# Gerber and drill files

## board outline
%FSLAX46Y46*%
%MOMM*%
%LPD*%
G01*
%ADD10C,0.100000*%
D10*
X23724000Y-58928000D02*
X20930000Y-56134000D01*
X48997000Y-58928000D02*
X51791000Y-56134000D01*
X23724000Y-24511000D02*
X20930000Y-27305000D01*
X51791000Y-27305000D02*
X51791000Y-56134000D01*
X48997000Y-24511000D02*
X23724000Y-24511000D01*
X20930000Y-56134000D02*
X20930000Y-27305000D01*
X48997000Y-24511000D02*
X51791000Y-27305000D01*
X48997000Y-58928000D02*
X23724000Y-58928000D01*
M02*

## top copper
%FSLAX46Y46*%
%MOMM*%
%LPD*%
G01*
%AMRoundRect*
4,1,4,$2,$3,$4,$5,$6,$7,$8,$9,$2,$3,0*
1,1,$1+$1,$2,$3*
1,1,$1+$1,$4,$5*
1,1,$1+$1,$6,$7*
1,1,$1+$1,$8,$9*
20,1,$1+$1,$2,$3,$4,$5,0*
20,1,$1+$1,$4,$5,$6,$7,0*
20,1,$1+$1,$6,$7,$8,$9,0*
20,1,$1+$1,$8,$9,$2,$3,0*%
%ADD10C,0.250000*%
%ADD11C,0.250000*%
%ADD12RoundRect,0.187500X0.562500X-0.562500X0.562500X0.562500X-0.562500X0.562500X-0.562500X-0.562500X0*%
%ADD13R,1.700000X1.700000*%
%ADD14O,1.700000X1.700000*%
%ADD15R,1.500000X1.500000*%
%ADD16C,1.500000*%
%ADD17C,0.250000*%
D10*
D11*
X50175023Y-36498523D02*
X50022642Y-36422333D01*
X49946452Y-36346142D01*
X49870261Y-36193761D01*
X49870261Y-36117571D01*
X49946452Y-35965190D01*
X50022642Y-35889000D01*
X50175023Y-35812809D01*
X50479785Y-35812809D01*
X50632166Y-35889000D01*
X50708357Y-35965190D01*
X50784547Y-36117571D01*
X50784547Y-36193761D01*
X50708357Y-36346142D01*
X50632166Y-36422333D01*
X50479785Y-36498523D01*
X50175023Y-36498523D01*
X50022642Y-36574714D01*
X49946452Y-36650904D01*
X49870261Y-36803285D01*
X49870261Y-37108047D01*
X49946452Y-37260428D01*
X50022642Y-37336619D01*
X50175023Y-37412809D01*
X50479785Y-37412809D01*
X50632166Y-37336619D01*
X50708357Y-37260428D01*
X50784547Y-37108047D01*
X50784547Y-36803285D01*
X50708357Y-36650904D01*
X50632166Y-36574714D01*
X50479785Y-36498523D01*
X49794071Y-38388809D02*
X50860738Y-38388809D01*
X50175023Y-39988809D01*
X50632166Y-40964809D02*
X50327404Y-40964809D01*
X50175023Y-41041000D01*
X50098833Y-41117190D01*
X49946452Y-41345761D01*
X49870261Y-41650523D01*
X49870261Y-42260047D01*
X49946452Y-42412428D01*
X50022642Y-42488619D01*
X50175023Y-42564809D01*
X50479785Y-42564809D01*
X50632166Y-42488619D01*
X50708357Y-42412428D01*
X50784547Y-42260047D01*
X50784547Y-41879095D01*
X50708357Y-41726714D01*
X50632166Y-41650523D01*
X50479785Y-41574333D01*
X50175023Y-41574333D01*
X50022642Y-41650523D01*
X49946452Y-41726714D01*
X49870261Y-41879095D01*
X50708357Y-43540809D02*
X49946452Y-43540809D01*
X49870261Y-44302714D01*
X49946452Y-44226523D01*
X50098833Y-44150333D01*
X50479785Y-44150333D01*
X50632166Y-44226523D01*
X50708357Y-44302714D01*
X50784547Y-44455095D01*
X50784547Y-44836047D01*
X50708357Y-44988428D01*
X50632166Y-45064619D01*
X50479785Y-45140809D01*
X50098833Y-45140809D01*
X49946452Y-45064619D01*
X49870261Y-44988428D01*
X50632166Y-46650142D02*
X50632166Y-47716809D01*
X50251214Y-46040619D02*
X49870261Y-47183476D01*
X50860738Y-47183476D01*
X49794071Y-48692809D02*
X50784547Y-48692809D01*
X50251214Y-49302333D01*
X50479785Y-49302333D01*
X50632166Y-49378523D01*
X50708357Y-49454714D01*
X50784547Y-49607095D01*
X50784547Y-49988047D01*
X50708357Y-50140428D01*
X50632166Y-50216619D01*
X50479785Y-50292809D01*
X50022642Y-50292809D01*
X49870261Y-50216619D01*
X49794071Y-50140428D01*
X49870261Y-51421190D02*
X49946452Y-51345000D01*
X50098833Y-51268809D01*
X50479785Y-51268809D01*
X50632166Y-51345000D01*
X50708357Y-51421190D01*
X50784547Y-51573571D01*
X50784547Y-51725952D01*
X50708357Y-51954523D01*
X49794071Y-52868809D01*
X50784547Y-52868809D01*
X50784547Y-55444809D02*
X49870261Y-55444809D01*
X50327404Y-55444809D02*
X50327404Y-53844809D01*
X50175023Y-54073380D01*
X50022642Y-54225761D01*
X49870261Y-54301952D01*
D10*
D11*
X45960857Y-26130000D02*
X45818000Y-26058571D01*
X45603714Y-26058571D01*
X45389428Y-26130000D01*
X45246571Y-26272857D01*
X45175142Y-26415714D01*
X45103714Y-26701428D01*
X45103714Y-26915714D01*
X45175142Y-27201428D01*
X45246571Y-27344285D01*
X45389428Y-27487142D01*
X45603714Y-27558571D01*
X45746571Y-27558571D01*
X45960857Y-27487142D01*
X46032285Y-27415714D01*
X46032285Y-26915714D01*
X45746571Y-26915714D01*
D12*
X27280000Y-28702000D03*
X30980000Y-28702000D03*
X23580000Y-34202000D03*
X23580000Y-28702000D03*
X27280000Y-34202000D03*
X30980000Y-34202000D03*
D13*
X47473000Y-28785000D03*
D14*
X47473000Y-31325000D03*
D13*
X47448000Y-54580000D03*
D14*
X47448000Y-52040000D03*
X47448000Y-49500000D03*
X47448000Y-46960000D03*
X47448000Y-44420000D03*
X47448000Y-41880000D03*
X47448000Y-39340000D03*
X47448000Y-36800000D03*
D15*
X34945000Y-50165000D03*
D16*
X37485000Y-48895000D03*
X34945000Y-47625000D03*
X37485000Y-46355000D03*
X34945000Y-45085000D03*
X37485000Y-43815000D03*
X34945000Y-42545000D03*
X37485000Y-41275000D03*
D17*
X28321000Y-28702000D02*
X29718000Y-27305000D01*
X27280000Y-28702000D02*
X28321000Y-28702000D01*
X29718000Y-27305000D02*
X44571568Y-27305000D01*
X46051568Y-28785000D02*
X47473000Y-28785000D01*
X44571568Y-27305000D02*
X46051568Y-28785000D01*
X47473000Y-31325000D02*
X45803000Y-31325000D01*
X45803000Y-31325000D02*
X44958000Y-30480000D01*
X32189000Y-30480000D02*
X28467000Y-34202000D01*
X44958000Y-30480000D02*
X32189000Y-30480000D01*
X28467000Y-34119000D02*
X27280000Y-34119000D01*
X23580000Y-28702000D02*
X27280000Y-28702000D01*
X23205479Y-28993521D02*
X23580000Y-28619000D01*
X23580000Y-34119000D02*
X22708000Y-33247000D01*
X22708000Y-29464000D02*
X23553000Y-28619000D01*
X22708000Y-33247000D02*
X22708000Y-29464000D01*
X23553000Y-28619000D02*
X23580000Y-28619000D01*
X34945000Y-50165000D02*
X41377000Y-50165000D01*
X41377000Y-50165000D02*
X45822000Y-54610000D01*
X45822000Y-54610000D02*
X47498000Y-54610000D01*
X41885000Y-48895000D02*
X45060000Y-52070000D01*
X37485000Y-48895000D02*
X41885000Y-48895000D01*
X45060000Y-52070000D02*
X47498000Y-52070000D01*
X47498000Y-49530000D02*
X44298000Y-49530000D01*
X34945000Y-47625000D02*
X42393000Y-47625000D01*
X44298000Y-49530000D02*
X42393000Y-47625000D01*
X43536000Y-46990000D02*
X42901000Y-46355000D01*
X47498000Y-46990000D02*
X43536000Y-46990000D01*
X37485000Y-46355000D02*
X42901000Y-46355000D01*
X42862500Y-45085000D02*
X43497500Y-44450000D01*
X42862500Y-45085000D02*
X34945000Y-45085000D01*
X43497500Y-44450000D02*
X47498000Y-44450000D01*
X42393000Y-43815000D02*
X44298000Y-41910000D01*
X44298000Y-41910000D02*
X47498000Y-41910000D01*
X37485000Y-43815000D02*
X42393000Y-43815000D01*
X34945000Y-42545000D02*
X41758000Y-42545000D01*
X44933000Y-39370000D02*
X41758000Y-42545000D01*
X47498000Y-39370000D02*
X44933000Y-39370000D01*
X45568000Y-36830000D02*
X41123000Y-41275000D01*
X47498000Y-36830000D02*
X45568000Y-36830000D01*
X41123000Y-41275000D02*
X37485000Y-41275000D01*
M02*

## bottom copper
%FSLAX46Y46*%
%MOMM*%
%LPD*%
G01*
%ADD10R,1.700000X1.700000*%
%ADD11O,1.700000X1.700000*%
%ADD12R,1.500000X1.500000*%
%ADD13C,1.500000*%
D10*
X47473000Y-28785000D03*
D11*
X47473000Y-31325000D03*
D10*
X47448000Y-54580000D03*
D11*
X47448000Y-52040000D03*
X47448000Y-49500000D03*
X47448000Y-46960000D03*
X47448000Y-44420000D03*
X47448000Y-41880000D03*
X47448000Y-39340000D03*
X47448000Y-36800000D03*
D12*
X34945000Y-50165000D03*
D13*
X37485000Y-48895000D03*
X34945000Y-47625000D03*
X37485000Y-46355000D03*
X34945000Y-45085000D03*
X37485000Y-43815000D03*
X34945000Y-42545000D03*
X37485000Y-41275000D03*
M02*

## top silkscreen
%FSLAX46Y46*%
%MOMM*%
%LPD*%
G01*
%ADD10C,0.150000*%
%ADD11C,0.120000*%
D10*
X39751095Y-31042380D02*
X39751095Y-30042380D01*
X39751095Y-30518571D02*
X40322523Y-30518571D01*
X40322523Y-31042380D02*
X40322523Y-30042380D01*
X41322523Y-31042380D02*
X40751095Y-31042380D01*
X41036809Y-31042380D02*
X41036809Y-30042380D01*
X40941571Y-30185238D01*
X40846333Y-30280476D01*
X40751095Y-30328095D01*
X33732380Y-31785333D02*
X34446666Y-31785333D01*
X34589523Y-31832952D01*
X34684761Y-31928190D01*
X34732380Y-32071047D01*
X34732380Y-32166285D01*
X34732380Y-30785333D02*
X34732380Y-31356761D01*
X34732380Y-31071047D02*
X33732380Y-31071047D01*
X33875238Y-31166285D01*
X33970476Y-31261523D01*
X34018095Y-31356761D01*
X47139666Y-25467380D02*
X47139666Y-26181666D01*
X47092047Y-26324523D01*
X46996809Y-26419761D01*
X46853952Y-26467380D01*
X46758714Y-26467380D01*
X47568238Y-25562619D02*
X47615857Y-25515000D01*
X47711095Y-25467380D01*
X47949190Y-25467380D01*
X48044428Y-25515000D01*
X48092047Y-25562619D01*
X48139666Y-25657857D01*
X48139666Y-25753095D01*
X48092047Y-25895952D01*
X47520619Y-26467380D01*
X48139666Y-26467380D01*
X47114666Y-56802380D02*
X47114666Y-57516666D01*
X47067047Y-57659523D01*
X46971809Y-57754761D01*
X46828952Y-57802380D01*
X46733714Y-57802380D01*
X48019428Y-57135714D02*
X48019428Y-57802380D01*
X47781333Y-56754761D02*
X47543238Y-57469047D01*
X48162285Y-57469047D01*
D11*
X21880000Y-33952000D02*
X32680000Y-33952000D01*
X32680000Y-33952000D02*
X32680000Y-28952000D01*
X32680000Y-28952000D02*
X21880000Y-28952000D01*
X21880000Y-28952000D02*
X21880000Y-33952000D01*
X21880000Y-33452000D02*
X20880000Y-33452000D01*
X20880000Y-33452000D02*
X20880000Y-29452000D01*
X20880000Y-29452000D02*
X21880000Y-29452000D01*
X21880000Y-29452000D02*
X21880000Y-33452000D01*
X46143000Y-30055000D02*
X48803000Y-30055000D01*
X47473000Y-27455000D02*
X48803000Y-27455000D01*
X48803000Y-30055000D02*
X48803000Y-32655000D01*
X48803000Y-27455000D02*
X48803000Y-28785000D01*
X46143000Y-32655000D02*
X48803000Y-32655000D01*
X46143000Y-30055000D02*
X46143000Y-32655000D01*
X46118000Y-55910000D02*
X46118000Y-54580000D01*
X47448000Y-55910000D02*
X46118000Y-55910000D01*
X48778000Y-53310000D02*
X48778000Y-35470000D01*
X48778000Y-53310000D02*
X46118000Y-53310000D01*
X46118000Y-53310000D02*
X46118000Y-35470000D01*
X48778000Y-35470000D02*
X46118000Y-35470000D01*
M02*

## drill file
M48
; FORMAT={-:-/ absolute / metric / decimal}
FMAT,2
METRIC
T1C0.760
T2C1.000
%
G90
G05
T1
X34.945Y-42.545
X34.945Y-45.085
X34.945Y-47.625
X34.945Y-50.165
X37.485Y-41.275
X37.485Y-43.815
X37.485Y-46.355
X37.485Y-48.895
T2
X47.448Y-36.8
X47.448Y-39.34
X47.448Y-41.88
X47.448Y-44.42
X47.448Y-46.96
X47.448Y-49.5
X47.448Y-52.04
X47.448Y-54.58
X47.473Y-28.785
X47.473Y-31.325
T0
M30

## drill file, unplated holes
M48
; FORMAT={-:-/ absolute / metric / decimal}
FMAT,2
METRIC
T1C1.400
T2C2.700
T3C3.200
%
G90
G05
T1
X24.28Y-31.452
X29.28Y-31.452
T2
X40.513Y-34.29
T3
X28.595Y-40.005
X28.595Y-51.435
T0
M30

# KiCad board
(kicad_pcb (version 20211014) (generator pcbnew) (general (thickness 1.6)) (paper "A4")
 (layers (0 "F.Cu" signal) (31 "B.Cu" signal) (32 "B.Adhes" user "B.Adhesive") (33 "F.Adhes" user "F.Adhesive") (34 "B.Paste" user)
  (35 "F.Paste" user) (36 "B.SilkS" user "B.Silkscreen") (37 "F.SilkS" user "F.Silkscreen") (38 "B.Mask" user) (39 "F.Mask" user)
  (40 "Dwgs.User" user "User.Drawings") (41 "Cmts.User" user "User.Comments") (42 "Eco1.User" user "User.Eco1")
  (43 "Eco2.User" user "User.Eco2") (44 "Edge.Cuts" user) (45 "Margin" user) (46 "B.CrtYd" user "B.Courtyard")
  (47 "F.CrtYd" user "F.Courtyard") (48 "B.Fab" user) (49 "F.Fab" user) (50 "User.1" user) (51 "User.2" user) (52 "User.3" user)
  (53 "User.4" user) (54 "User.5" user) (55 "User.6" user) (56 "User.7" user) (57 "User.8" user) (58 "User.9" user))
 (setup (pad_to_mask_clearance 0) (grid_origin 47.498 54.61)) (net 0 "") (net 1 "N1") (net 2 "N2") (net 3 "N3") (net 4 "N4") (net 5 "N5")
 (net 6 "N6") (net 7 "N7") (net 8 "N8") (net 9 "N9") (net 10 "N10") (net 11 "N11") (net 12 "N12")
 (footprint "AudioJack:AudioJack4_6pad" (layer "F.Cu") (at 27.28 31.452 90)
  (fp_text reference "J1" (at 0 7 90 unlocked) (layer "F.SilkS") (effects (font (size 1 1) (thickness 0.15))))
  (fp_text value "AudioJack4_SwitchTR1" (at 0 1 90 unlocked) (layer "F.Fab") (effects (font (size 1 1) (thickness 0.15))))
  (fp_rect (start -2.5 -5.4) (end 2.5 5.4) (layer "F.SilkS") (width 0.12) (fill none))
  (fp_rect (start -2 -5.4) (end 2 -6.4) (layer "F.SilkS") (width 0.12) (fill none))
  (pad "" np_thru_hole circle (at 0 -3 90) (size 1.4 1.4) (drill 1.4) (layers F&B.Cu *.Mask))
  (pad "" np_thru_hole circle (at 0 2 90) (size 1.4 1.4) (drill 1.4) (layers F&B.Cu *.Mask))
  (pad "R1" smd roundrect (at 2.75 0 90) (size 1.5 1.5) (layers "F.Cu" "F.Paste" "F.Mask") (roundrect_rratio 0.125) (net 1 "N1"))
  (pad "R1N" smd roundrect (at 2.75 3.7 90) (size 1.5 1.5) (layers "F.Cu" "F.Paste" "F.Mask") (roundrect_rratio 0.125) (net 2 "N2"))
  (pad "R2" smd roundrect (at -2.75 -3.7 90) (size 1.5 1.5) (layers "F.Cu" "F.Paste" "F.Mask") (roundrect_rratio 0.125) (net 1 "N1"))
  (pad "S" smd roundrect (at 2.75 -3.7 90) (size 1.5 1.5) (layers "F.Cu" "F.Paste" "F.Mask") (roundrect_rratio 0.125) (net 1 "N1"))
  (pad "T" smd roundrect (at -2.75 0 90) (size 1.5 1.5) (layers "F.Cu" "F.Paste" "F.Mask") (roundrect_rratio 0.125) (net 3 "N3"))
  (pad "TN" smd roundrect (at -2.75 3.7 90) (size 1.5 1.5) (layers "F.Cu" "F.Paste" "F.Mask") (roundrect_rratio 0.125) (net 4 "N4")))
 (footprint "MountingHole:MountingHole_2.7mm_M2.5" (layer "F.Cu") (at 40.513 34.29)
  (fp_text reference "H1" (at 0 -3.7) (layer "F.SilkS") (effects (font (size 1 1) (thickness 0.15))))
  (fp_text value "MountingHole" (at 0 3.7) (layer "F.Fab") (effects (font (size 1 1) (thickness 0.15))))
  (pad "" np_thru_hole circle locked (at 0 0) (size 2.7 2.7) (drill 2.7) (layers *.Cu *.Mask)))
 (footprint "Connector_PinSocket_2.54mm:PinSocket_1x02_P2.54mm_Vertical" (layer "F.Cu") (at 47.473 28.785)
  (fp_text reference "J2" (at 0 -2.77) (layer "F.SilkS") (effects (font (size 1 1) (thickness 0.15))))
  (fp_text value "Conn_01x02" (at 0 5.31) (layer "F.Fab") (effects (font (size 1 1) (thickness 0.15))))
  (fp_line (start -1.33 1.27) (end 1.33 1.27) (layer "F.SilkS") (width 0.12))
  (fp_line (start 0 -1.33) (end 1.33 -1.33) (layer "F.SilkS") (width 0.12))
  (fp_line (start 1.33 1.27) (end 1.33 3.87) (layer "F.SilkS") (width 0.12))
  (fp_line (start 1.33 -1.33) (end 1.33 0) (layer "F.SilkS") (width 0.12))
  (fp_line (start -1.33 3.87) (end 1.33 3.87) (layer "F.SilkS") (width 0.12))
  (fp_line (start -1.33 1.27) (end -1.33 3.87) (layer "F.SilkS") (width 0.12))
  (pad "1" thru_hole rect locked (at 0 0) (size 1.7 1.7) (drill 1) (layers *.Cu *.Mask) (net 1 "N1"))
  (pad "2" thru_hole oval locked (at 0 2.54) (size 1.7 1.7) (drill 1) (layers *.Cu *.Mask) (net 3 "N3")))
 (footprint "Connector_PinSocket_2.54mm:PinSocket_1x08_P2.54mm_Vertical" (layer "F.Cu") (at 47.448 54.58 180)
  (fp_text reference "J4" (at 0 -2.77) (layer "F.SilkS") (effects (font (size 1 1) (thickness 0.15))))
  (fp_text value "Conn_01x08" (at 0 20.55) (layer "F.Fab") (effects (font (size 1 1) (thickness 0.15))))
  (fp_line (start 1.33 -1.33) (end 1.33 0) (layer "F.SilkS") (width 0.12))
  (fp_line (start 0 -1.33) (end 1.33 -1.33) (layer "F.SilkS") (width 0.12))
  (fp_line (start -1.33 1.27) (end -1.33 19.11) (layer "F.SilkS") (width 0.12))
  (fp_line (start -1.33 1.27) (end 1.33 1.27) (layer "F.SilkS") (width 0.12))
  (fp_line (start 1.33 1.27) (end 1.33 19.11) (layer "F.SilkS") (width 0.12))
  (fp_line (start -1.33 19.11) (end 1.33 19.11) (layer "F.SilkS") (width 0.12))
  (pad "1" thru_hole rect locked (at 0 0 180) (size 1.7 1.7) (drill 1) (layers *.Cu *.Mask) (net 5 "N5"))
  (pad "2" thru_hole oval locked (at 0 2.54 180) (size 1.7 1.7) (drill 1) (layers *.Cu *.Mask) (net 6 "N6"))
  (pad "3" thru_hole oval locked (at 0 5.08 180) (size 1.7 1.7) (drill 1) (layers *.Cu *.Mask) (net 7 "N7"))
  (pad "4" thru_hole oval locked (at 0 7.62 180) (size 1.7 1.7) (drill 1) (layers *.Cu *.Mask) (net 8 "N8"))
  (pad "5" thru_hole oval locked (at 0 10.16 180) (size 1.7 1.7) (drill 1) (layers *.Cu *.Mask) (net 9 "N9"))
  (pad "6" thru_hole oval locked (at 0 12.7 180) (size 1.7 1.7) (drill 1) (layers *.Cu *.Mask) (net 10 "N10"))
  (pad "7" thru_hole oval locked (at 0 15.24 180) (size 1.7 1.7) (drill 1) (layers *.Cu *.Mask) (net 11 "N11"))
  (pad "8" thru_hole oval locked (at 0 17.78 180) (size 1.7 1.7) (drill 1) (layers *.Cu *.Mask) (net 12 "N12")))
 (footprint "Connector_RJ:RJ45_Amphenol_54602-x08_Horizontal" (layer "B.Cu") (at 34.945 50.165 90)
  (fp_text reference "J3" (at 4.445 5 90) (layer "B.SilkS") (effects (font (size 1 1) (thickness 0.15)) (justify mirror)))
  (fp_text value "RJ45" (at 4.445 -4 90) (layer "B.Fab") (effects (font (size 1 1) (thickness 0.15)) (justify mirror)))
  (pad "" np_thru_hole circle locked (at 10.16 -6.35 90) (size 3.2 3.2) (drill 3.2) (layers *.Cu *.Mask))
  (pad "" np_thru_hole circle locked (at -1.27 -6.35 90) (size 3.2 3.2) (drill 3.2) (layers *.Cu *.Mask))
  (pad "1" thru_hole rect locked (at 0 0 90) (size 1.5 1.5) (drill 0.76) (layers *.Cu *.Mask) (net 5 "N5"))
  (pad "2" thru_hole circle locked (at 1.27 2.54 90) (size 1.5 1.5) (drill 0.76) (layers *.Cu *.Mask) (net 6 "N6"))
  (pad "3" thru_hole circle locked (at 2.54 0 90) (size 1.5 1.5) (drill 0.76) (layers *.Cu *.Mask) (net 7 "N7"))
  (pad "4" thru_hole circle locked (at 3.81 2.54 90) (size 1.5 1.5) (drill 0.76) (layers *.Cu *.Mask) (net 8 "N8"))
  (pad "5" thru_hole circle locked (at 5.08 0 90) (size 1.5 1.5) (drill 0.76) (layers *.Cu *.Mask) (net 9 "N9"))
  (pad "6" thru_hole circle locked (at 6.35 2.54 90) (size 1.5 1.5) (drill 0.76) (layers *.Cu *.Mask) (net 10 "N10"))
  (pad "7" thru_hole circle locked (at 7.62 0 90) (size 1.5 1.5) (drill 0.76) (layers *.Cu *.Mask) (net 11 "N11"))
  (pad "8" thru_hole circle locked (at 8.89 2.54 90) (size 1.5 1.5) (drill 0.76) (layers *.Cu *.Mask) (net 12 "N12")))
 (gr_line (start 23.724 58.928) (end 20.93 56.134) (layer "Edge.Cuts") (width 0.1))
 (gr_line (start 48.997 58.928) (end 51.791 56.134) (layer "Edge.Cuts") (width 0.1))
 (gr_line (start 23.724 24.511) (end 20.93 27.305) (layer "Edge.Cuts") (width 0.1))
 (gr_line (start 51.791 27.305) (end 51.791 56.134) (layer "Edge.Cuts") (width 0.1))
 (gr_line (start 48.997 24.511) (end 23.724 24.511) (layer "Edge.Cuts") (width 0.1))
 (gr_line (start 20.93 56.134) (end 20.93 27.305) (layer "Edge.Cuts") (width 0.1))
 (gr_line (start 48.997 24.511) (end 51.791 27.305) (layer "Edge.Cuts") (width 0.1))
 (gr_line (start 48.997 58.928) (end 23.724 58.928) (layer "Edge.Cuts") (width 0.1))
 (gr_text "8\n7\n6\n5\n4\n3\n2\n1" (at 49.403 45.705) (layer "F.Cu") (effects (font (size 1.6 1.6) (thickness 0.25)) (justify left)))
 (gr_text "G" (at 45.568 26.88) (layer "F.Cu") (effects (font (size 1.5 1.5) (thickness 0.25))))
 (segment (start 44.958 30.48) (end 32.189 30.48) (width 0.25) (layer "F.Cu") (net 3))
 (segment (start 32.189 30.48) (end 28.467 34.202) (width 0.25) (layer "F.Cu") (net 3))
 (segment (start 47.473 31.325) (end 45.803 31.325) (width 0.25) (layer "F.Cu") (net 3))
 (segment (start 45.803 31.325) (end 44.958 30.48) (width 0.25) (layer "F.Cu") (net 3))
 (segment (start 28.467 34.119) (end 27.28 34.119) (width 0.25) (layer "F.Cu") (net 3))
 (segment (start 28.321 28.702) (end 29.718 27.305) (width 0.25) (layer "F.Cu") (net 1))
 (segment (start 23.58 28.702) (end 27.28 28.702) (width 0.25) (layer "F.Cu") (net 1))
 (segment (start 23.205479 28.993521) (end 23.58 28.619) (width 0.25) (layer "F.Cu") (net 1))
 (segment (start 29.718 27.305) (end 44.571568 27.305) (width 0.25) (layer "F.Cu") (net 1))
 (segment (start 23.58 34.119) (end 22.708 33.247) (width 0.25) (layer "F.Cu") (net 1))
 (segment (start 22.708 29.464) (end 23.553 28.619) (width 0.25) (layer "F.Cu") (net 1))
 (segment (start 44.571568 27.305) (end 46.051568 28.785) (width 0.25) (layer "F.Cu") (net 1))
 (segment (start 46.051568 28.785) (end 47.473 28.785) (width 0.25) (layer "F.Cu") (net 1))
 (segment (start 27.28 28.702) (end 28.321 28.702) (width 0.25) (layer "F.Cu") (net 1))
 (segment (start 22.708 33.247) (end 22.708 29.464) (width 0.25) (layer "F.Cu") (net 1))
 (segment (start 23.553 28.619) (end 23.58 28.619) (width 0.25) (layer "F.Cu") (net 1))
 (segment (start 34.945 50.165) (end 41.377 50.165) (width 0.25) (layer "F.Cu") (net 5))
 (segment (start 41.377 50.165) (end 45.822 54.61) (width 0.25) (layer "F.Cu") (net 5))
 (segment (start 45.822 54.61) (end 47.498 54.61) (width 0.25) (layer "F.Cu") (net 5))
 (segment (start 41.885 48.895) (end 45.06 52.07) (width 0.25) (layer "F.Cu") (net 6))
 (segment (start 37.485 48.895) (end 41.885 48.895) (width 0.25) (layer "F.Cu") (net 6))
 (segment (start 45.06 52.07) (end 47.498 52.07) (width 0.25) (layer "F.Cu") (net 6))
 (segment (start 47.498 49.53) (end 44.298 49.53) (width 0.25) (layer "F.Cu") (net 7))
 (segment (start 34.945 47.625) (end 42.393 47.625) (width 0.25) (layer "F.Cu") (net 7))
 (segment (start 44.298 49.53) (end 42.393 47.625) (width 0.25) (layer "F.Cu") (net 7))
 (segment (start 43.536 46.99) (end 42.901 46.355) (width 0.25) (layer "F.Cu") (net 8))
 (segment (start 47.498 46.99) (end 43.536 46.99) (width 0.25) (layer "F.Cu") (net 8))
 (segment (start 37.485 46.355) (end 42.901 46.355) (width 0.25) (layer "F.Cu") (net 8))
 (segment (start 42.8625 45.085) (end 43.4975 44.45) (width 0.25) (layer "F.Cu") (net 9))
 (segment (start 42.8625 45.085) (end 34.945 45.085) (width 0.25) (layer "F.Cu") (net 9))
 (segment (start 43.4975 44.45) (end 47.498 44.45) (width 0.25) (layer "F.Cu") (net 9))
 (segment (start 42.393 43.815) (end 44.298 41.91) (width 0.25) (layer "F.Cu") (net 10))
 (segment (start 44.298 41.91) (end 47.498 41.91) (width 0.25) (layer "F.Cu") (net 10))
 (segment (start 37.485 43.815) (end 42.393 43.815) (width 0.25) (layer "F.Cu") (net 10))
 (segment (start 34.945 42.545) (end 41.758 42.545) (width 0.25) (layer "F.Cu") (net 11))
 (segment (start 44.933 39.37) (end 41.758 42.545) (width 0.25) (layer "F.Cu") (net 11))
 (segment (start 47.498 39.37) (end 44.933 39.37) (width 0.25) (layer "F.Cu") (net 11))
 (segment (start 45.568 36.83) (end 41.123 41.275) (width 0.25) (layer "F.Cu") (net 12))
 (segment (start 47.498 36.83) (end 45.568 36.83) (width 0.25) (layer "F.Cu") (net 12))
 (segment (start 41.123 41.275) (end 37.485 41.275) (width 0.25) (layer "F.Cu") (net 12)))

